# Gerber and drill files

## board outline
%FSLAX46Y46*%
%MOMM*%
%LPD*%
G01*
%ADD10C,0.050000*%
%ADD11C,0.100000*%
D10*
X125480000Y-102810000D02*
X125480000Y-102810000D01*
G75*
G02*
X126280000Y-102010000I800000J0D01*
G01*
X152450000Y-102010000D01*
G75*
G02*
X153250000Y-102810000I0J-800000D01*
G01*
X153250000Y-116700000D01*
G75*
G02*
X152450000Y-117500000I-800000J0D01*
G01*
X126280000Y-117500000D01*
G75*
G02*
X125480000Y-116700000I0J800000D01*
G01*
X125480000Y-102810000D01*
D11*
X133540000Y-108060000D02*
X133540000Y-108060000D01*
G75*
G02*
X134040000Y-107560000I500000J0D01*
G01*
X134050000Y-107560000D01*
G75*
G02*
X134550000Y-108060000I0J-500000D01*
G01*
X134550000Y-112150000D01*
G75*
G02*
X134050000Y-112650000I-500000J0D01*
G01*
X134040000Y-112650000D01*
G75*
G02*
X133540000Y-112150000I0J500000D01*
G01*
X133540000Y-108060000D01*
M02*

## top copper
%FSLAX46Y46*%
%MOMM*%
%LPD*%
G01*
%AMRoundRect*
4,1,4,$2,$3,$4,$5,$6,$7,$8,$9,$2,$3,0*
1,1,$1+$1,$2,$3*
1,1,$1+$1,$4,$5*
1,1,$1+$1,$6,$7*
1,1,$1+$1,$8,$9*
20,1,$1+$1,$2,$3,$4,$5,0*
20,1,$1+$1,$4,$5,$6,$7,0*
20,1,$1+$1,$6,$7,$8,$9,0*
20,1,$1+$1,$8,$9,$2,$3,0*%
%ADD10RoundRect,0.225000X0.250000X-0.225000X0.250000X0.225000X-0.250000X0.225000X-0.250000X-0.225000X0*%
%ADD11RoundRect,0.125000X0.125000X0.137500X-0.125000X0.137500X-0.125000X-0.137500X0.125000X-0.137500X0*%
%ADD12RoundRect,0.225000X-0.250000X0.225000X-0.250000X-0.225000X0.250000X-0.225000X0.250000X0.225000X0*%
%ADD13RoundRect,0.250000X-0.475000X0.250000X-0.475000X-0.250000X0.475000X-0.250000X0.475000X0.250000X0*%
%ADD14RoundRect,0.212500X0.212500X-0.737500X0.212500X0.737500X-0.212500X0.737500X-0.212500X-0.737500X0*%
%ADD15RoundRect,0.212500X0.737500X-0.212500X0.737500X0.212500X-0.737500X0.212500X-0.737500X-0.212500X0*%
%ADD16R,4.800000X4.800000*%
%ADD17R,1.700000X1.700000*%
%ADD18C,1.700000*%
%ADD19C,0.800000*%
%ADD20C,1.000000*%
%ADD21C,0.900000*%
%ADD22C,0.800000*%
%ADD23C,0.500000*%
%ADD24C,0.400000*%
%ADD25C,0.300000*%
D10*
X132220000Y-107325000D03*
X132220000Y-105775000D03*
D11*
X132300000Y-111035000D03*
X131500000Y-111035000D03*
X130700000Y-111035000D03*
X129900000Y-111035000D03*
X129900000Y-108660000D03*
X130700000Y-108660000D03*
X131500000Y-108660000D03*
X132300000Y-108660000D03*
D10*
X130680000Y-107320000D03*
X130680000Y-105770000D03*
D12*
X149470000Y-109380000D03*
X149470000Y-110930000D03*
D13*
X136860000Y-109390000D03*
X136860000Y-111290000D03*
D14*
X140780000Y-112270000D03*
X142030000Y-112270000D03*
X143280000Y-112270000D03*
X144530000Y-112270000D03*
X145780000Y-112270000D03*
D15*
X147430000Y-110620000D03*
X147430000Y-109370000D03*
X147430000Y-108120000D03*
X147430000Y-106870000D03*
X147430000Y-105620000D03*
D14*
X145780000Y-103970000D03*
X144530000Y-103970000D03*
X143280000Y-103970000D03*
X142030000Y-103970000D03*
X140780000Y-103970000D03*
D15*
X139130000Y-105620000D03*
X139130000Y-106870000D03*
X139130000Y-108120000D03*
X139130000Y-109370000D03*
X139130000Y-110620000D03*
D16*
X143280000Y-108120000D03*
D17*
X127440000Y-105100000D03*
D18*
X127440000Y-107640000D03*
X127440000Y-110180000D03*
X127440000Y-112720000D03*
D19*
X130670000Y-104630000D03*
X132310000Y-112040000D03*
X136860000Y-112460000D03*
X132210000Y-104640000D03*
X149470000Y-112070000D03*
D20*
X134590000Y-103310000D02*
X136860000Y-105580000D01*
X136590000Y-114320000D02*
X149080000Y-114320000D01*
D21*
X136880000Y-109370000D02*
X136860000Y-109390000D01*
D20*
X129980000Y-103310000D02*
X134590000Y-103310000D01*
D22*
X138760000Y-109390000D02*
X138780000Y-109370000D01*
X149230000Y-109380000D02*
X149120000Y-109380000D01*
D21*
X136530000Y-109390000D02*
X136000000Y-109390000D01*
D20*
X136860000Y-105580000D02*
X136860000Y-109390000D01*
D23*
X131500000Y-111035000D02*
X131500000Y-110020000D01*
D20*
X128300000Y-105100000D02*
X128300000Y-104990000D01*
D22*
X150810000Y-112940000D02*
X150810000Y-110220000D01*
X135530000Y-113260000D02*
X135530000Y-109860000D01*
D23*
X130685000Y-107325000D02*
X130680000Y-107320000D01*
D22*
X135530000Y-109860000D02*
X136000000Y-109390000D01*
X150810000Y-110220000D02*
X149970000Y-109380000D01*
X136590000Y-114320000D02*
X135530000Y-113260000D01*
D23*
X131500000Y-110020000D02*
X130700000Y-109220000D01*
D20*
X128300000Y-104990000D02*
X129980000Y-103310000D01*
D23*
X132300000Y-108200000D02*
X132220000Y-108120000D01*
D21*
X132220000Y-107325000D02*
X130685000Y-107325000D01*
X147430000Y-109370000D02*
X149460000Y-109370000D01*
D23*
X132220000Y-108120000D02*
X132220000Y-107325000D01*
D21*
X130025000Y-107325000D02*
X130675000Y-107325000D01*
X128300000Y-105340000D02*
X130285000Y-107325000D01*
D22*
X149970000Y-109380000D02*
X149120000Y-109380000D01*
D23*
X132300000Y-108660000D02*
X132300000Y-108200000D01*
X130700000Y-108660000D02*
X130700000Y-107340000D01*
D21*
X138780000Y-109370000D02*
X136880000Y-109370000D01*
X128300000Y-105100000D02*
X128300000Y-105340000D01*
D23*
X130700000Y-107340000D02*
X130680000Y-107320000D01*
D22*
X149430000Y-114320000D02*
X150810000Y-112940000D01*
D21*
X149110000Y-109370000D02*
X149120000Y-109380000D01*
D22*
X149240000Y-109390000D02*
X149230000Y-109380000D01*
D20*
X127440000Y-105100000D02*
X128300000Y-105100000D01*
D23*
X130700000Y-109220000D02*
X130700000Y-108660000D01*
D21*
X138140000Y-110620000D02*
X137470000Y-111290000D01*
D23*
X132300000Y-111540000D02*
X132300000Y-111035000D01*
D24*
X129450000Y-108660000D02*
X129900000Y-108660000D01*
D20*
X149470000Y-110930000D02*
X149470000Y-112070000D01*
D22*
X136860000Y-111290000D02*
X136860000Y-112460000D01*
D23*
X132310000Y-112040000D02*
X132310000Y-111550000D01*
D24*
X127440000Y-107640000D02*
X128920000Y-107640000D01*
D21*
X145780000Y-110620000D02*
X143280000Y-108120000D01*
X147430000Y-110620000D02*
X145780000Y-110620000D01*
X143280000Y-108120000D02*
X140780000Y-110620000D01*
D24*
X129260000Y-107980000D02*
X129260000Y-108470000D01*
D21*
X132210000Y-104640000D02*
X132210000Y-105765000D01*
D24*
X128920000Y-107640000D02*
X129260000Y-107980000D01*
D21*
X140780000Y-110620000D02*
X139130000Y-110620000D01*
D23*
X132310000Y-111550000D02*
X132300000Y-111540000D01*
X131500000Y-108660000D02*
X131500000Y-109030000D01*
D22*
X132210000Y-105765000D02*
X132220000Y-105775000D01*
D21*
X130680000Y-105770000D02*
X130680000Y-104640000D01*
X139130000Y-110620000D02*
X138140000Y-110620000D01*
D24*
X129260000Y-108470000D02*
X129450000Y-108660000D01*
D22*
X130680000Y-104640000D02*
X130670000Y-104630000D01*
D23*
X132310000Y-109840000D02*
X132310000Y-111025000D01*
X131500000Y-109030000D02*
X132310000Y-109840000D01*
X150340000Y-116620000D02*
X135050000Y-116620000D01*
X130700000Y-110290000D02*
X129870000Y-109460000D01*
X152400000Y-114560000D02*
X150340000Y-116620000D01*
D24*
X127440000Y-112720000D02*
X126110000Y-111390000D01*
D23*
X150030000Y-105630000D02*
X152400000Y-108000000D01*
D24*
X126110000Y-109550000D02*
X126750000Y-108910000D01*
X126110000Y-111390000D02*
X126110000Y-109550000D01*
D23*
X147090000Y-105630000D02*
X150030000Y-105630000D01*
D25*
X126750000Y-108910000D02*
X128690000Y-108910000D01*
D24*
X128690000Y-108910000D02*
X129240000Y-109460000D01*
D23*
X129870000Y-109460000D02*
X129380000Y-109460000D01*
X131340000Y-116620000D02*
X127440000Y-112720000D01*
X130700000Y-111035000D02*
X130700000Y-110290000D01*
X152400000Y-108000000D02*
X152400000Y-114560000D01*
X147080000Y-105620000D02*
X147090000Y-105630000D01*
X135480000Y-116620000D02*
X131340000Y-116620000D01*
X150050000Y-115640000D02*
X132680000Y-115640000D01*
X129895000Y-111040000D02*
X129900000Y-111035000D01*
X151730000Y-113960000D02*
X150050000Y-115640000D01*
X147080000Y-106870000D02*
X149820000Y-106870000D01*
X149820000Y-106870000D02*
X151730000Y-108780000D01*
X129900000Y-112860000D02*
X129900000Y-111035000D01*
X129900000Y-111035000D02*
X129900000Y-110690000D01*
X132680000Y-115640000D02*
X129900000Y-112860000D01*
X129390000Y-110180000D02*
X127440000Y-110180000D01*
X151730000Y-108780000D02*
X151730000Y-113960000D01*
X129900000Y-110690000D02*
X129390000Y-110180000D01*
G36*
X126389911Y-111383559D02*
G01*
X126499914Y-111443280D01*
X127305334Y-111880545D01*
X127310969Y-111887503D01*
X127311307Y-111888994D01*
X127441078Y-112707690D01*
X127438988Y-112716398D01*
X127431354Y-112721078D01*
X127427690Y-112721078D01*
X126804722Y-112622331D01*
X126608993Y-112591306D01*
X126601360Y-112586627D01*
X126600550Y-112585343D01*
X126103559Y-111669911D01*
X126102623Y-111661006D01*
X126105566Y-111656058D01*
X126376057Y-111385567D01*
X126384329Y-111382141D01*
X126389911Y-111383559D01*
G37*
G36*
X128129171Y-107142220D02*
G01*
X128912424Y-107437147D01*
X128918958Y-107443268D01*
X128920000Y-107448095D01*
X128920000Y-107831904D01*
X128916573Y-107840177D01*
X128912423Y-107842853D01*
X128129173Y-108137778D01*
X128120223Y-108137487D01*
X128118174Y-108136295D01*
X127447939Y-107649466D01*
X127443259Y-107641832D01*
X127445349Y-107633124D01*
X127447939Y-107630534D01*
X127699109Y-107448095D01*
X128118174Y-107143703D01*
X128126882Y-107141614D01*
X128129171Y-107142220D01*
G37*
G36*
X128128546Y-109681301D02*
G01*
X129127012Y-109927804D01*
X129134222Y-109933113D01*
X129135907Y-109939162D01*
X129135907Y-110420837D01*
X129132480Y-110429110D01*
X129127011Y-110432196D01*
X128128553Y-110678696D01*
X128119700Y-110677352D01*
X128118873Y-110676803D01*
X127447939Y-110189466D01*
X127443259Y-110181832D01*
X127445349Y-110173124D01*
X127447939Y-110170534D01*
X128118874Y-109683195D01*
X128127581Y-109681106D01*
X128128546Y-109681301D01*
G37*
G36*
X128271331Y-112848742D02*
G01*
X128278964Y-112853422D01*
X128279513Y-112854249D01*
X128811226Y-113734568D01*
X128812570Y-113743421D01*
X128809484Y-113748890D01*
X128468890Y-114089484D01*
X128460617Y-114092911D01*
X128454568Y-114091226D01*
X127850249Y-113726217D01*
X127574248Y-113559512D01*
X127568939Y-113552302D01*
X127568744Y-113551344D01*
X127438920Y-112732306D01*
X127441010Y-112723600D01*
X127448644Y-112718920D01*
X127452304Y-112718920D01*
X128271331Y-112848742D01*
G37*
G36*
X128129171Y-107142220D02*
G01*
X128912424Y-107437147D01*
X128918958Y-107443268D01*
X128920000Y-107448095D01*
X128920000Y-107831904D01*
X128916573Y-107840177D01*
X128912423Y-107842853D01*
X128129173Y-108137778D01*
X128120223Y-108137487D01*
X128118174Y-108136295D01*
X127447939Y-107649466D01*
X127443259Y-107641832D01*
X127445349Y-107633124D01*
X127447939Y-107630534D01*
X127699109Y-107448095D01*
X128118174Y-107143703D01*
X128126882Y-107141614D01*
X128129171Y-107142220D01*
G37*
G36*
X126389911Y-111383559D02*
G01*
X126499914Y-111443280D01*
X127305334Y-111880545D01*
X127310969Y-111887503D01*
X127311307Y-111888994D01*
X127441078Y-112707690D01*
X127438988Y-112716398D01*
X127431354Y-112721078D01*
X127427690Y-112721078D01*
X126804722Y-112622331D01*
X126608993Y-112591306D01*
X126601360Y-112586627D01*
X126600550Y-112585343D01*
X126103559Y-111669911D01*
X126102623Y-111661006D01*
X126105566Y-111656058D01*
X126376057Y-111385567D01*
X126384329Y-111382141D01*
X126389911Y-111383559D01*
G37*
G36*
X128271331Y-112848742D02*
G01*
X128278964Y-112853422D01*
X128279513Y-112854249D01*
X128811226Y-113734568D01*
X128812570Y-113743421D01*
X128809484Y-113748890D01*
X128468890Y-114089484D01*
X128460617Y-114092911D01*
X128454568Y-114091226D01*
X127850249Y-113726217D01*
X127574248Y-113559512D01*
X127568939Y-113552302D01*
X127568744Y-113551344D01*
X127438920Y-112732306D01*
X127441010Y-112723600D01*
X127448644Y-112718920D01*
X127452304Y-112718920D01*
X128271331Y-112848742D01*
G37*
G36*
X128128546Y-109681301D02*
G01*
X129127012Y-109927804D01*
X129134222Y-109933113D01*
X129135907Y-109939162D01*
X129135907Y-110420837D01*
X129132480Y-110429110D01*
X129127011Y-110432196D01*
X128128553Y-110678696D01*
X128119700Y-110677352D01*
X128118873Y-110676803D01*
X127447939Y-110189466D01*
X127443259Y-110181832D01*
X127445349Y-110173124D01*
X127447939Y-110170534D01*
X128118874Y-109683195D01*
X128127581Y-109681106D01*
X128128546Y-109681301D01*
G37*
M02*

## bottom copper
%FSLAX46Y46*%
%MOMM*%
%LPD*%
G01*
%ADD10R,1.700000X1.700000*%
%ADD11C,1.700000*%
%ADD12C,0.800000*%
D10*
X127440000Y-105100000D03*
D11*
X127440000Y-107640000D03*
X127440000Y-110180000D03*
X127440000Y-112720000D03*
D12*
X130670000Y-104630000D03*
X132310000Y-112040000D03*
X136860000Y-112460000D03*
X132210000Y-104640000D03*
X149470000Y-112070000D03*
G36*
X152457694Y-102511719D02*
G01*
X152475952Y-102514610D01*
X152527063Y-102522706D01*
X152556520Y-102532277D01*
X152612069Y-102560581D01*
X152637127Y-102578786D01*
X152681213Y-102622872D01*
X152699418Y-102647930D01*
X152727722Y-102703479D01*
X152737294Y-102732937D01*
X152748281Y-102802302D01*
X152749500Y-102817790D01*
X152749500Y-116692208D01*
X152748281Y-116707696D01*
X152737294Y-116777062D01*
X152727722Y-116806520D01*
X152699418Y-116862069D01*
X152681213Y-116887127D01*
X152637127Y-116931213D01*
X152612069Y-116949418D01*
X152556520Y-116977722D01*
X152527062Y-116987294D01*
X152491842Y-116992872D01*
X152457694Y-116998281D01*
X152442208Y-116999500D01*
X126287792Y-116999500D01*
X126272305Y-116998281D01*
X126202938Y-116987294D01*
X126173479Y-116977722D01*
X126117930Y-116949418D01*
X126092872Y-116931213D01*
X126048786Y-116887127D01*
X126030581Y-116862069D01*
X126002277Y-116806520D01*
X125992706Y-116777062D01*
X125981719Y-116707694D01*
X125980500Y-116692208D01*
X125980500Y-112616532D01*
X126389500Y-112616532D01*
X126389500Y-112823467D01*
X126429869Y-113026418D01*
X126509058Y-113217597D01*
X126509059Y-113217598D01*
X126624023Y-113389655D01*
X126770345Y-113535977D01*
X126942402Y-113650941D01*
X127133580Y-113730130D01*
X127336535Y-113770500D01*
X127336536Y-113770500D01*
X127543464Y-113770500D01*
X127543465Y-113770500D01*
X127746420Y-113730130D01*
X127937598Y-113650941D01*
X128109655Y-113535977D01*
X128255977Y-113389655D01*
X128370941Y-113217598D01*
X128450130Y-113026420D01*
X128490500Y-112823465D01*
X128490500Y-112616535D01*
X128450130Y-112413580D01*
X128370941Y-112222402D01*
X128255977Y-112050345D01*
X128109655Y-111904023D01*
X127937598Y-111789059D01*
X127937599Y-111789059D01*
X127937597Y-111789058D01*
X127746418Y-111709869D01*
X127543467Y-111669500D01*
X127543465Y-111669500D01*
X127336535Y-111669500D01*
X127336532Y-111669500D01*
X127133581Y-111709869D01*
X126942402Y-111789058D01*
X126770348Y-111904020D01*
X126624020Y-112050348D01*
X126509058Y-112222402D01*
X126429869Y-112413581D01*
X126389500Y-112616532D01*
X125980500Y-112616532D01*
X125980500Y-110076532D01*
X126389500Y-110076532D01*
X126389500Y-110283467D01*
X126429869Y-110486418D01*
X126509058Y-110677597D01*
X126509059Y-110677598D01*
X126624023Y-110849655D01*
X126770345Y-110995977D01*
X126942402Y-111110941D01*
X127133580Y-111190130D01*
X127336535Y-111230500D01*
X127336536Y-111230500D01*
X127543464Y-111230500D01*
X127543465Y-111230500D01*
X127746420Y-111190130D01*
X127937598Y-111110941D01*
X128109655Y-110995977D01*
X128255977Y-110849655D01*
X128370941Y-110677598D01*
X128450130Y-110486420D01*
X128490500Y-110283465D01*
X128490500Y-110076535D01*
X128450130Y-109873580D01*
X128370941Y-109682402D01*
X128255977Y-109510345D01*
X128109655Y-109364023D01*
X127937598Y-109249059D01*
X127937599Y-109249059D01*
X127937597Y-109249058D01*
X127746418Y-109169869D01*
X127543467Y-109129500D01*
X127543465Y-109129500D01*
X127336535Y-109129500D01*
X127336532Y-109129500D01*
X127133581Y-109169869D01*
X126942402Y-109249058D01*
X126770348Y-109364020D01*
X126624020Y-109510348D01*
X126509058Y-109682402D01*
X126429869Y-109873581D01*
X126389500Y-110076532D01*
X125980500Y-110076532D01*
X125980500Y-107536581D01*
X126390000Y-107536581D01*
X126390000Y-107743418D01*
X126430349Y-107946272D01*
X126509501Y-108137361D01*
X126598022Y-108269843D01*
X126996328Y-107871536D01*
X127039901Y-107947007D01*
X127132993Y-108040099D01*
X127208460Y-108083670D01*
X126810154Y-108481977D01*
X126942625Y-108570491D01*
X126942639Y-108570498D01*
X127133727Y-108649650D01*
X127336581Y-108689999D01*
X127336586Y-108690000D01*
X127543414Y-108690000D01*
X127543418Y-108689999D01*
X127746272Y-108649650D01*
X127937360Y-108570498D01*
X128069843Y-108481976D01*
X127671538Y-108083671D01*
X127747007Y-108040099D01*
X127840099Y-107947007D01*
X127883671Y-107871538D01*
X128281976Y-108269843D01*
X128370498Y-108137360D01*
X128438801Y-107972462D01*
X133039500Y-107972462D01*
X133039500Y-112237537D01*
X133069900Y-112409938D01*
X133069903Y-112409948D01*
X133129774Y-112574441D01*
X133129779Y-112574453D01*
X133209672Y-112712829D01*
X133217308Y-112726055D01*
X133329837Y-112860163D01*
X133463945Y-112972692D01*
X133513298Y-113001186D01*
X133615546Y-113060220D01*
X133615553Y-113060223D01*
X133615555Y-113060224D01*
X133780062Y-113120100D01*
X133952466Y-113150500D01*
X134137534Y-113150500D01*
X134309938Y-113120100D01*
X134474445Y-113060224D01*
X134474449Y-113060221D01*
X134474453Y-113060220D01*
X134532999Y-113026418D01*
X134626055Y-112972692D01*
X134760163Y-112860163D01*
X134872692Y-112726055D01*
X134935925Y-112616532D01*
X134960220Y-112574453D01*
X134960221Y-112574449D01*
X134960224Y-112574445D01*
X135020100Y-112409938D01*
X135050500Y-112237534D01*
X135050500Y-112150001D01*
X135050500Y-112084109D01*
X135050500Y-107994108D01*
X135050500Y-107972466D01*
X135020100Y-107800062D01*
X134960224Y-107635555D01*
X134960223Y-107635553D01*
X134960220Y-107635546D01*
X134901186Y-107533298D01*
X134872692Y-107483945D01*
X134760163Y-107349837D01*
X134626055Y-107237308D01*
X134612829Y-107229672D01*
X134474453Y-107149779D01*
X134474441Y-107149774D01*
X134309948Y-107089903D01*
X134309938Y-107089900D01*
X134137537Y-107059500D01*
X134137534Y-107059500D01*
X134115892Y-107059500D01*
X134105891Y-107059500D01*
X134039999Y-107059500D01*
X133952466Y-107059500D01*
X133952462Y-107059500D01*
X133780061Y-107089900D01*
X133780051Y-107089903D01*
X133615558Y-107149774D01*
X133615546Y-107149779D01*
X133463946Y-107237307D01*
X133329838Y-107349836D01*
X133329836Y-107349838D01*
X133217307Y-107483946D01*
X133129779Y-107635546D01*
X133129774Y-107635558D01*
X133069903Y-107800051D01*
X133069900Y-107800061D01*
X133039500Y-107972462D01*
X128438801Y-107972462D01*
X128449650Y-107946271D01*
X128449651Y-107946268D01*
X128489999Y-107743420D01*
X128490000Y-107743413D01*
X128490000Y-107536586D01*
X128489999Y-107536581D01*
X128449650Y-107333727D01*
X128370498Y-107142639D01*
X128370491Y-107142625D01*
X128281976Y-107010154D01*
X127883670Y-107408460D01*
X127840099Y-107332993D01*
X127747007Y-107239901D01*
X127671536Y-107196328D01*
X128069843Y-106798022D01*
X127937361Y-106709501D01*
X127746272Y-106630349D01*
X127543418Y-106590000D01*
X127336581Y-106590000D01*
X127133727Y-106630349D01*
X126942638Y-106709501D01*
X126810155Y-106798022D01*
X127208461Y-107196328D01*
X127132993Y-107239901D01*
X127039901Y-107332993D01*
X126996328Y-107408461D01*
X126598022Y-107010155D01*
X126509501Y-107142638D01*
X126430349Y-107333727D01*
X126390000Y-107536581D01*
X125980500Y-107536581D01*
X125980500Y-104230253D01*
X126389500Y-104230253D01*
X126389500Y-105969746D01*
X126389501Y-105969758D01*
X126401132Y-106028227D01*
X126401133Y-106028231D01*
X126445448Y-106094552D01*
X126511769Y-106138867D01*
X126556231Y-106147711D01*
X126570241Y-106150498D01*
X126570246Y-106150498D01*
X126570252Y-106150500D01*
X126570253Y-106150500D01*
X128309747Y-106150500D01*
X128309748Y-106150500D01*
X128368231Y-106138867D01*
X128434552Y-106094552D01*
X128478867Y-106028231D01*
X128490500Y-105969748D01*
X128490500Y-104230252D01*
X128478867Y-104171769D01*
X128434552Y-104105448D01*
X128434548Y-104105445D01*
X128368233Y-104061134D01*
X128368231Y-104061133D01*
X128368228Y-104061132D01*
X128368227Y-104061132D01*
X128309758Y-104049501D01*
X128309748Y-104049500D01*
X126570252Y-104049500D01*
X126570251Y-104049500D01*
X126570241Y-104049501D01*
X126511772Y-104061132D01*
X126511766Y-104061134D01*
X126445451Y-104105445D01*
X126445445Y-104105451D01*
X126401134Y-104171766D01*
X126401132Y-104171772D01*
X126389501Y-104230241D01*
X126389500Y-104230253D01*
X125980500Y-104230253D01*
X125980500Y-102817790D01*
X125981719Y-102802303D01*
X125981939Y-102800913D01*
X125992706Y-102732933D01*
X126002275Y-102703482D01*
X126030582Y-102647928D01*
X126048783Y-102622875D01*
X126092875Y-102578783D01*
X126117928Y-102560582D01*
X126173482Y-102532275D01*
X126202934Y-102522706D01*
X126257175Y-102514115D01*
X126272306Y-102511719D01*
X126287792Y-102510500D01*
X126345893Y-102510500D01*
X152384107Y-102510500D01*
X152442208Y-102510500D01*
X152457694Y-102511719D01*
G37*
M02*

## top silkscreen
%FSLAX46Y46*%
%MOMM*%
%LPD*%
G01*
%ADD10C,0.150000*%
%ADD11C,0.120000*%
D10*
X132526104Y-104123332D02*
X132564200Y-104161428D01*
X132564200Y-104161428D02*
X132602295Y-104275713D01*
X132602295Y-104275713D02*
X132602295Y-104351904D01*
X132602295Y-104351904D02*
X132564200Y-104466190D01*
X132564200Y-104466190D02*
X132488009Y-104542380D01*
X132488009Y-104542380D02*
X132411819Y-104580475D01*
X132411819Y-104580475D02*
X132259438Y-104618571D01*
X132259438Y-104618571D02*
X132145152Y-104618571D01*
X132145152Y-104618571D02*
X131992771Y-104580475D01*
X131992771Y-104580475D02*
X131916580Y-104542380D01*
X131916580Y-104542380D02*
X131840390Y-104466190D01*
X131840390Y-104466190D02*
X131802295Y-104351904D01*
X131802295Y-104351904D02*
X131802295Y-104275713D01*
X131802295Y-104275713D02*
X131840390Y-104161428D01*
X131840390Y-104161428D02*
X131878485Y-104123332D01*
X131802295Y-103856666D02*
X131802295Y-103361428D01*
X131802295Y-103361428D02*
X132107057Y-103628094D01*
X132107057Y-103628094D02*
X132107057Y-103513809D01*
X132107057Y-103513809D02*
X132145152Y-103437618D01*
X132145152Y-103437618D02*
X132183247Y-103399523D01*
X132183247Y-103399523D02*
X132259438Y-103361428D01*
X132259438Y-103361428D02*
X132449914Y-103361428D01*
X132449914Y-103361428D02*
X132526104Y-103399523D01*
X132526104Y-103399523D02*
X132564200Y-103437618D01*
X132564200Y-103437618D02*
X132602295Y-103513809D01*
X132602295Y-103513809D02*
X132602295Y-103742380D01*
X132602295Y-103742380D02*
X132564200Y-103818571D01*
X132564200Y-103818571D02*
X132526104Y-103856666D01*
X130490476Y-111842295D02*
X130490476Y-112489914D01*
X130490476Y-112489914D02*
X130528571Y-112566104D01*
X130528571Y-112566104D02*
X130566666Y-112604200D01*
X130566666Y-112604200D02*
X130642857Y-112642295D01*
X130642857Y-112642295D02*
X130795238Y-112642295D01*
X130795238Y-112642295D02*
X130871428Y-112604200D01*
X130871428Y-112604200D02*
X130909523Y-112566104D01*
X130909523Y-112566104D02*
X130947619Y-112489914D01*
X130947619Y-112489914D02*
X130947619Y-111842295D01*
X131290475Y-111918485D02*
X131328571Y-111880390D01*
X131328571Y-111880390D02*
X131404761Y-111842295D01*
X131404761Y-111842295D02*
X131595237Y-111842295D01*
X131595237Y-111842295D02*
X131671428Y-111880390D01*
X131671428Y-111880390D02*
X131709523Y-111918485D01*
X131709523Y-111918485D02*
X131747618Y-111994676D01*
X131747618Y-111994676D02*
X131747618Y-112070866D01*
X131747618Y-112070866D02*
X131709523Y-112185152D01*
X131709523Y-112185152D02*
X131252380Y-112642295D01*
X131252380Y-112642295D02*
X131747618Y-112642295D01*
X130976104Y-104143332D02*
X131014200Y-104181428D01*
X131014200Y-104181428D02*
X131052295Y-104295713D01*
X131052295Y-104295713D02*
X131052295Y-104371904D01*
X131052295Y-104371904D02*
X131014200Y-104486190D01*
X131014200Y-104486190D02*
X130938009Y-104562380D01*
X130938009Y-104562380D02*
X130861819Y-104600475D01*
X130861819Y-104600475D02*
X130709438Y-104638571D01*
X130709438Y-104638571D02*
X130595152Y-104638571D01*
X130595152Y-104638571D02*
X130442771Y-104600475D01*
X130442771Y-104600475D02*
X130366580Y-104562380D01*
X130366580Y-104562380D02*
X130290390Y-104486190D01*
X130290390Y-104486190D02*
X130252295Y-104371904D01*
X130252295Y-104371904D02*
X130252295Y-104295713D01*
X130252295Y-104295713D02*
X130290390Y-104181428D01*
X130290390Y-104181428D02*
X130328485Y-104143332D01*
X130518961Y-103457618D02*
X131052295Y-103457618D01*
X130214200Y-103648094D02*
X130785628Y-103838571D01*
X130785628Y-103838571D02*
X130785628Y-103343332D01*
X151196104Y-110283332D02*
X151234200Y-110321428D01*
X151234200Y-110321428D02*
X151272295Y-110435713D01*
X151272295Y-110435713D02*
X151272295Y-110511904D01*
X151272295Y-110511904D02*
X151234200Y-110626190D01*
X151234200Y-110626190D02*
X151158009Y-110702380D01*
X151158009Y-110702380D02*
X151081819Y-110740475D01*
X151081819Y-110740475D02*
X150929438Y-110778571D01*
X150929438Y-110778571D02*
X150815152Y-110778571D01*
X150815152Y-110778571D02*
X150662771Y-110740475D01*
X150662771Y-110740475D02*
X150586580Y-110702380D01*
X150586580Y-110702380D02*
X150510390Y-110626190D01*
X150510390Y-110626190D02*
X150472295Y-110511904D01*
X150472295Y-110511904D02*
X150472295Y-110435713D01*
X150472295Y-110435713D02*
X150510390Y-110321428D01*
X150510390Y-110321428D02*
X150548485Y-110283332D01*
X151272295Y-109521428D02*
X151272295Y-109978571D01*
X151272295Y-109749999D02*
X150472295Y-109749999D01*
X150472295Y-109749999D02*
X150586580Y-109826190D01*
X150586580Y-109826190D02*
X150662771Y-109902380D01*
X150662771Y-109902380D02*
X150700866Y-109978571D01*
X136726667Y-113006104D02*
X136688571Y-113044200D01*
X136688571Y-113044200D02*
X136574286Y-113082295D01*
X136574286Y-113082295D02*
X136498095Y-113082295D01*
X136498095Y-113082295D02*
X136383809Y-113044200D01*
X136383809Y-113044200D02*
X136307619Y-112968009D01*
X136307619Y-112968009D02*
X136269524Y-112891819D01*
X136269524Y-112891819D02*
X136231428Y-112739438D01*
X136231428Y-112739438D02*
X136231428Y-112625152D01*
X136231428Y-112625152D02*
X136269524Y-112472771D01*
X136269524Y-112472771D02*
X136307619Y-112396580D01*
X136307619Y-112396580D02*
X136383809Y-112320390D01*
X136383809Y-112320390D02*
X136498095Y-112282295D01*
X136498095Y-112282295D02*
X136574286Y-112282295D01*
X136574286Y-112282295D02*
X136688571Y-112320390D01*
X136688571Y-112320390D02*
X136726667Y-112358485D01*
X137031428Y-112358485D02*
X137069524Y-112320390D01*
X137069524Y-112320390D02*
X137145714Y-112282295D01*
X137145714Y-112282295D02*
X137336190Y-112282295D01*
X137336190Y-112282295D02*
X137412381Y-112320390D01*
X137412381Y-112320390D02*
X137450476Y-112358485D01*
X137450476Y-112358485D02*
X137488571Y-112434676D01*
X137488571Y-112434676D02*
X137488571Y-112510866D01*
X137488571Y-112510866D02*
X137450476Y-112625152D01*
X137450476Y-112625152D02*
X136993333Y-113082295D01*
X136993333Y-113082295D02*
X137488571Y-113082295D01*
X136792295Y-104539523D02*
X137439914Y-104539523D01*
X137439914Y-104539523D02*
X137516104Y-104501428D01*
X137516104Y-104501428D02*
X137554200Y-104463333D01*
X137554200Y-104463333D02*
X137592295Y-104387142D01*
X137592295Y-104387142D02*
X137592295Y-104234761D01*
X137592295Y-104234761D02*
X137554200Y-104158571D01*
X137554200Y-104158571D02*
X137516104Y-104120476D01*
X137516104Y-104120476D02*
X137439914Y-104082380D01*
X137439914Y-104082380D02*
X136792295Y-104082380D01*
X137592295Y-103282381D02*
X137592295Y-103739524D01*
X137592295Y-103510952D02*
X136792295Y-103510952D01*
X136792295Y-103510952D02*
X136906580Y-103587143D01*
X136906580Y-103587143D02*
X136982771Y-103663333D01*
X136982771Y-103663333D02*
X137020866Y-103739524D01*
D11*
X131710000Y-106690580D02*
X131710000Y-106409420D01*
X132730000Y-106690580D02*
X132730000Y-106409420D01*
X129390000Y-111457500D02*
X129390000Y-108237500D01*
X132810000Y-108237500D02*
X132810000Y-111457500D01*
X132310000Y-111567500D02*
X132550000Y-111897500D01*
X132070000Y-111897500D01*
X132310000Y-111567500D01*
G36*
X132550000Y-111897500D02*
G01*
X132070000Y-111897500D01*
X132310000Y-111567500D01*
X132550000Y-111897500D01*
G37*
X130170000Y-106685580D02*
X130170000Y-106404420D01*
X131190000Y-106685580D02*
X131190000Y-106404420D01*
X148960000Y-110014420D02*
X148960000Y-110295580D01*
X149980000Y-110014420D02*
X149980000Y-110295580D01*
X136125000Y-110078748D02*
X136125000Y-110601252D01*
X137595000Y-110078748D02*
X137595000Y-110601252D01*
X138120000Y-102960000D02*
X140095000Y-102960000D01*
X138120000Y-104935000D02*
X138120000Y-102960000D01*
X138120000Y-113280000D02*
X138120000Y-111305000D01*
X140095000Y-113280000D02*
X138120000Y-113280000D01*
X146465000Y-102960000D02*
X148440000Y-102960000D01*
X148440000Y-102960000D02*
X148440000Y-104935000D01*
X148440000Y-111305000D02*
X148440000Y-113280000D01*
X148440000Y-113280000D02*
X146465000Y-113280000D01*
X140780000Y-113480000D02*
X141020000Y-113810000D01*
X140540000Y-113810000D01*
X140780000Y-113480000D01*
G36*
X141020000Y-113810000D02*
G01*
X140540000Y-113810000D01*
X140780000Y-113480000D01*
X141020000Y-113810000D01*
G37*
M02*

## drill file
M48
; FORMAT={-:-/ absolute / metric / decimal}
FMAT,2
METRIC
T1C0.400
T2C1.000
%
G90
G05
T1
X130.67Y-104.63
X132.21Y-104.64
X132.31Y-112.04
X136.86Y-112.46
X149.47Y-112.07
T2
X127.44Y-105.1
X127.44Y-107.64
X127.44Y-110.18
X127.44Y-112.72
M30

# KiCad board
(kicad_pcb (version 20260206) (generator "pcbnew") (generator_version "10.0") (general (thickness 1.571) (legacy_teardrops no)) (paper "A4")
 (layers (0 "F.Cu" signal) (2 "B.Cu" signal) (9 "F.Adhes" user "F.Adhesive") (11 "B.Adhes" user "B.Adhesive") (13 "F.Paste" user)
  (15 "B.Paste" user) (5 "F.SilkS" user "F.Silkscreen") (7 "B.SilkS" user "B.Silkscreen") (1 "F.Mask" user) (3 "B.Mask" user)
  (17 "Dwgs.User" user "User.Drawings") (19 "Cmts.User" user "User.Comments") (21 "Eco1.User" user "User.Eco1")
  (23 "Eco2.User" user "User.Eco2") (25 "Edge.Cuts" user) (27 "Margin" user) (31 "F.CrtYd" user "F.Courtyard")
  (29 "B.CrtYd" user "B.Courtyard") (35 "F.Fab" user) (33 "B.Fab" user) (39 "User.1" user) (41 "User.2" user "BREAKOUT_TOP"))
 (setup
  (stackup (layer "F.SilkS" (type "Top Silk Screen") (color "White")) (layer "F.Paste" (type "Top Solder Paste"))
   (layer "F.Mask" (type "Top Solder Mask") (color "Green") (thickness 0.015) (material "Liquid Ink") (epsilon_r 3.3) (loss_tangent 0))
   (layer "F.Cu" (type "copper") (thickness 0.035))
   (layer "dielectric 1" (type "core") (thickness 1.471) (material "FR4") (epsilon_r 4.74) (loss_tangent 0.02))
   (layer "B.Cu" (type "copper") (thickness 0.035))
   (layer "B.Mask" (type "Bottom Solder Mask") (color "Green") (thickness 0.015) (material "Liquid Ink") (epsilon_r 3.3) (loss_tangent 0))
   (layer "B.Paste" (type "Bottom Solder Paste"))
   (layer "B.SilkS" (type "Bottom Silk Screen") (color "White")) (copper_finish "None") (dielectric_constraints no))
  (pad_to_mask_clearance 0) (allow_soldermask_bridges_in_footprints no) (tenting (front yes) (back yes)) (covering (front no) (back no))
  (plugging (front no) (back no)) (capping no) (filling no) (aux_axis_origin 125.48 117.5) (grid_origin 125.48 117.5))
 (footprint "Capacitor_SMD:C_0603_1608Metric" (layer "F.Cu") (at 132.22 106.55 90)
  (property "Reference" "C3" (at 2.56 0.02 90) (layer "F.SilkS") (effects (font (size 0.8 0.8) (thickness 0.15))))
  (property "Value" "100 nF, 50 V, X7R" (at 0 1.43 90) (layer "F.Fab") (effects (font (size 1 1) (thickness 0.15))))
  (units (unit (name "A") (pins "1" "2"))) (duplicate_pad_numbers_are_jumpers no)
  (fp_line (start -0.14058 -0.51) (end 0.14058 -0.51) (stroke (width 0.12) (type solid)) (layer "F.SilkS"))
  (fp_line (start -0.14058 0.51) (end 0.14058 0.51) (stroke (width 0.12) (type solid)) (layer "F.SilkS"))
  (pad "1" smd roundrect (at -0.775 0 90) (size 0.9 0.95) (layers "F.Cu" "F.Mask" "F.Paste") (roundrect_rratio 0.25) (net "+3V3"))
  (pad "2" smd roundrect (at 0.775 0 90) (size 0.9 0.95) (layers "F.Cu" "F.Mask" "F.Paste") (roundrect_rratio 0.25) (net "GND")))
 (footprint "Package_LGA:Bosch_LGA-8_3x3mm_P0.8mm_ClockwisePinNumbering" (layer "F.Cu") (at 131.1 109.8475 180)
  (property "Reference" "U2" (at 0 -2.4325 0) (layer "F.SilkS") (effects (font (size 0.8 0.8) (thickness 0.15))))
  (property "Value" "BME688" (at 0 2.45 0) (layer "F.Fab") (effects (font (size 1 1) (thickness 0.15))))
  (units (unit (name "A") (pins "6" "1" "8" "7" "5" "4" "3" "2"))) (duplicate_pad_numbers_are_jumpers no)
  (fp_line (start 1.71 -1.61) (end 1.71 1.61) (stroke (width 0.12) (type solid)) (layer "F.SilkS"))
  (fp_line (start -1.71 1.61) (end -1.71 -1.61) (stroke (width 0.12) (type solid)) (layer "F.SilkS"))
  (fp_poly (pts (xy -1.21 -1.72) (xy -1.45 -2.05) (xy -0.97 -2.05)) (stroke (width 0.12) (type solid)) (fill yes) (layer "F.SilkS"))
  (pad "1" smd roundrect (at -1.2 -1.1875 180) (size 0.5 0.525) (layers "F.Cu" "F.Mask" "F.Paste") (roundrect_rratio 0.25) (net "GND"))
  (pad "2" smd roundrect (at -0.4 -1.1875 180) (size 0.5 0.525) (layers "F.Cu" "F.Mask" "F.Paste") (roundrect_rratio 0.25) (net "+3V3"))
  (pad "3" smd roundrect (at 0.4 -1.1875 180) (size 0.5 0.525) (layers "F.Cu" "F.Mask" "F.Paste") (roundrect_rratio 0.25) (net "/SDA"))
  (pad "4" smd roundrect (at 1.2 -1.1875 180) (size 0.5 0.525) (layers "F.Cu" "F.Mask" "F.Paste") (roundrect_rratio 0.25) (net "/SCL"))
  (pad "5" smd roundrect (at 1.2 1.1875 180) (size 0.5 0.525) (layers "F.Cu" "F.Mask" "F.Paste") (roundrect_rratio 0.25) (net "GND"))
  (pad "6" smd roundrect (at 0.4 1.1875 180) (size 0.5 0.525) (layers "F.Cu" "F.Mask" "F.Paste") (roundrect_rratio 0.25) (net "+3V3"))
  (pad "7" smd roundrect (at -0.4 1.1875 180) (size 0.5 0.525) (layers "F.Cu" "F.Mask" "F.Paste") (roundrect_rratio 0.25) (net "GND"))
  (pad "8" smd roundrect (at -1.2 1.1875 180) (size 0.5 0.525) (layers "F.Cu" "F.Mask" "F.Paste") (roundrect_rratio 0.25) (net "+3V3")))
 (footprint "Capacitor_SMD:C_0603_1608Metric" (layer "F.Cu") (at 130.68 106.545 90)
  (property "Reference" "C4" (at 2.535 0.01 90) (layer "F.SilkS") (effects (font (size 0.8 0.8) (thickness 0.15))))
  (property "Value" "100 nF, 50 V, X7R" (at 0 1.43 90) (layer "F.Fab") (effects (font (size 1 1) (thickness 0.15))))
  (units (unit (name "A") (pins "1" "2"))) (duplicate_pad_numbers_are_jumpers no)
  (fp_line (start -0.14058 -0.51) (end 0.14058 -0.51) (stroke (width 0.12) (type solid)) (layer "F.SilkS"))
  (fp_line (start -0.14058 0.51) (end 0.14058 0.51) (stroke (width 0.12) (type solid)) (layer "F.SilkS"))
  (pad "1" smd roundrect (at -0.775 0 90) (size 0.9 0.95) (layers "F.Cu" "F.Mask" "F.Paste") (roundrect_rratio 0.25) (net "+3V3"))
  (pad "2" smd roundrect (at 0.775 0 90) (size 0.9 0.95) (layers "F.Cu" "F.Mask" "F.Paste") (roundrect_rratio 0.25) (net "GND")))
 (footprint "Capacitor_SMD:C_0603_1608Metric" (layer "F.Cu") (at 149.47 110.155 -90)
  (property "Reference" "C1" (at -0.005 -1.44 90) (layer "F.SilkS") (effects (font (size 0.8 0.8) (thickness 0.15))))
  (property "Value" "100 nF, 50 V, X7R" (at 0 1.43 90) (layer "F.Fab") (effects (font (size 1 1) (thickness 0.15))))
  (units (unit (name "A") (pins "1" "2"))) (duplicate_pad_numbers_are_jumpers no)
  (fp_line (start -0.14058 0.51) (end 0.14058 0.51) (stroke (width 0.12) (type solid)) (layer "F.SilkS"))
  (fp_line (start -0.14058 -0.51) (end 0.14058 -0.51) (stroke (width 0.12) (type solid)) (layer "F.SilkS"))
  (pad "1" smd roundrect (at -0.775 0 270) (size 0.9 0.95) (layers "F.Cu" "F.Mask" "F.Paste") (roundrect_rratio 0.25) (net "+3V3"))
  (pad "2" smd roundrect (at 0.775 0 270) (size 0.9 0.95) (layers "F.Cu" "F.Mask" "F.Paste") (roundrect_rratio 0.25) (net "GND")))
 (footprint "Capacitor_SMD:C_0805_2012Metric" (layer "F.Cu") (at 136.86 110.34 -90)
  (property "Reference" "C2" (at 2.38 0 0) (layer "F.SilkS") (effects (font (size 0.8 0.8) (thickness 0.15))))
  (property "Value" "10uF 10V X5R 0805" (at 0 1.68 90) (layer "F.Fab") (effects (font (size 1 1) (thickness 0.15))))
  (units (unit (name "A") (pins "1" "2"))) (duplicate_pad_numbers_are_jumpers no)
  (fp_line (start -0.261252 0.735) (end 0.261252 0.735) (stroke (width 0.12) (type solid)) (layer "F.SilkS"))
  (fp_line (start -0.261252 -0.735) (end 0.261252 -0.735) (stroke (width 0.12) (type solid)) (layer "F.SilkS"))
  (pad "1" smd roundrect (at -0.95 0 270) (size 1 1.45) (layers "F.Cu" "F.Mask" "F.Paste") (roundrect_rratio 0.25) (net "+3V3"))
  (pad "2" smd roundrect (at 0.95 0 270) (size 1 1.45) (layers "F.Cu" "F.Mask" "F.Paste") (roundrect_rratio 0.25) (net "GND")))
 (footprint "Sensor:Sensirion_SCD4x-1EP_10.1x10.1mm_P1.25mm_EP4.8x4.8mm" (layer "F.Cu") (at 143.28 108.12 90)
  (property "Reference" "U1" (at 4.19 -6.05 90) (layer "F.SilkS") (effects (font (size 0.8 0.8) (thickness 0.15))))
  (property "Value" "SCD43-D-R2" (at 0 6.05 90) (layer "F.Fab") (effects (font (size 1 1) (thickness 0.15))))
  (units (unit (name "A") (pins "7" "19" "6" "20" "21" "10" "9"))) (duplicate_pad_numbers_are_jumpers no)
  (fp_line (start 5.16 -5.16) (end 5.16 -3.185) (stroke (width 0.12) (type solid)) (layer "F.SilkS"))
  (fp_line (start 3.185 -5.16) (end 5.16 -5.16) (stroke (width 0.12) (type solid)) (layer "F.SilkS"))
  (fp_line (start -5.16 -5.16) (end -3.185 -5.16) (stroke (width 0.12) (type solid)) (layer "F.SilkS"))
  (fp_line (start -5.16 -3.185) (end -5.16 -5.16) (stroke (width 0.12) (type solid)) (layer "F.SilkS"))
  (fp_line (start 5.16 3.185) (end 5.16 5.16) (stroke (width 0.12) (type solid)) (layer "F.SilkS"))
  (fp_line (start 5.16 5.16) (end 3.185 5.16) (stroke (width 0.12) (type solid)) (layer "F.SilkS"))
  (fp_line (start -3.185 5.16) (end -5.16 5.16) (stroke (width 0.12) (type solid)) (layer "F.SilkS"))
  (fp_line (start -5.16 5.16) (end -5.16 3.185) (stroke (width 0.12) (type solid)) (layer "F.SilkS"))
  (fp_poly (pts (xy -5.36 -2.5) (xy -5.69 -2.26) (xy -5.69 -2.74)) (stroke (width 0.12) (type solid)) (fill yes) (layer "F.SilkS"))
  (pad "" smd roundrect (at -1.2 -1.2 90) (size 1.93 1.93) (layers "F.Paste") (roundrect_rratio 0.129534))
  (pad "" smd roundrect (at -1.2 1.2 90) (size 1.93 1.93) (layers "F.Paste") (roundrect_rratio 0.129534))
  (pad "" smd roundrect (at 1.2 -1.2 90) (size 1.93 1.93) (layers "F.Paste") (roundrect_rratio 0.129534))
  (pad "" smd roundrect (at 1.2 1.2 90) (size 1.93 1.93) (layers "F.Paste") (roundrect_rratio 0.129534))
  (pad "1" smd roundrect (at -4.15 -2.5 90) (size 1.9 0.85) (layers "F.Cu" "F.Mask" "F.Paste") (roundrect_rratio 0.25))
  (pad "2" smd roundrect (at -4.15 -1.25 90) (size 1.9 0.85) (layers "F.Cu" "F.Mask" "F.Paste") (roundrect_rratio 0.25))
  (pad "3" smd roundrect (at -4.15 0 90) (size 1.9 0.85) (layers "F.Cu" "F.Mask" "F.Paste") (roundrect_rratio 0.25))
  (pad "4" smd roundrect (at -4.15 1.25 90) (size 1.9 0.85) (layers "F.Cu" "F.Mask" "F.Paste") (roundrect_rratio 0.25))
  (pad "5" smd roundrect (at -4.15 2.5 90) (size 1.9 0.85) (layers "F.Cu" "F.Mask" "F.Paste") (roundrect_rratio 0.25))
  (pad "6" smd roundrect (at -2.5 4.15 90) (size 0.85 1.9) (layers "F.Cu" "F.Mask" "F.Paste") (roundrect_rratio 0.25) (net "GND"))
  (pad "7" smd roundrect (at -1.25 4.15 90) (size 0.85 1.9) (layers "F.Cu" "F.Mask" "F.Paste") (roundrect_rratio 0.25) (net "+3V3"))
  (pad "8" smd roundrect (at 0 4.15 90) (size 0.85 1.9) (layers "F.Cu" "F.Mask" "F.Paste") (roundrect_rratio 0.25))
  (pad "9" smd roundrect (at 1.25 4.15 90) (size 0.85 1.9) (layers "F.Cu" "F.Mask" "F.Paste") (roundrect_rratio 0.25) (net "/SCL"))
  (pad "10" smd roundrect (at 2.5 4.15 90) (size 0.85 1.9) (layers "F.Cu" "F.Mask" "F.Paste") (roundrect_rratio 0.25) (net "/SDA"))
  (pad "11" smd roundrect (at 4.15 2.5 90) (size 1.9 0.85) (layers "F.Cu" "F.Mask" "F.Paste") (roundrect_rratio 0.25))
  (pad "12" smd roundrect (at 4.15 1.25 90) (size 1.9 0.85) (layers "F.Cu" "F.Mask" "F.Paste") (roundrect_rratio 0.25))
  (pad "13" smd roundrect (at 4.15 0 90) (size 1.9 0.85) (layers "F.Cu" "F.Mask" "F.Paste") (roundrect_rratio 0.25))
  (pad "14" smd roundrect (at 4.15 -1.25 90) (size 1.9 0.85) (layers "F.Cu" "F.Mask" "F.Paste") (roundrect_rratio 0.25))
  (pad "15" smd roundrect (at 4.15 -2.5 90) (size 1.9 0.85) (layers "F.Cu" "F.Mask" "F.Paste") (roundrect_rratio 0.25))
  (pad "16" smd roundrect (at 2.5 -4.15 90) (size 0.85 1.9) (layers "F.Cu" "F.Mask" "F.Paste") (roundrect_rratio 0.25))
  (pad "17" smd roundrect (at 1.25 -4.15 90) (size 0.85 1.9) (layers "F.Cu" "F.Mask" "F.Paste") (roundrect_rratio 0.25))
  (pad "18" smd roundrect (at 0 -4.15 90) (size 0.85 1.9) (layers "F.Cu" "F.Mask" "F.Paste") (roundrect_rratio 0.25))
  (pad "19" smd roundrect (at -1.25 -4.15 90) (size 0.85 1.9) (layers "F.Cu" "F.Mask" "F.Paste") (roundrect_rratio 0.25) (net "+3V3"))
  (pad "20" smd roundrect (at -2.5 -4.15 90) (size 0.85 1.9) (layers "F.Cu" "F.Mask" "F.Paste") (roundrect_rratio 0.25) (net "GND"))
  (pad "21" smd rect (at 0 0 90) (size 4.8 4.8) (layers "F.Cu" "F.Mask") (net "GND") (zone_connect 2)))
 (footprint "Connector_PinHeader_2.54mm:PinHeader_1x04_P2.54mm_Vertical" (layer "B.Cu") (at 127.44 105.1 180)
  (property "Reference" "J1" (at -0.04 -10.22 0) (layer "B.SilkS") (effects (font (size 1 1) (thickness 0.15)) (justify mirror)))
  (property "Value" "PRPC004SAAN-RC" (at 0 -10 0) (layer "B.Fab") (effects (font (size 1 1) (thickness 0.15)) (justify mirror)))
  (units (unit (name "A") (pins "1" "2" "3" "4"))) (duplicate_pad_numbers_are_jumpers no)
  (pad "1" thru_hole rect (at 0 0 180) (size 1.7 1.7) (drill 1) (layers "*.Cu" "*.Mask") (remove_unused_layers no) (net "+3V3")
   (teardrops (best_length_ratio 0.5) (max_length 1) (best_width_ratio 1) (max_width 1) (curved_edges no) (filter_ratio 0.9) (enabled yes)
    (allow_two_segments no) (prefer_zone_connections yes)))
  (pad "2" thru_hole circle (at 0 -2.54 180) (size 1.7 1.7) (drill 1) (layers "*.Cu" "*.Mask") (remove_unused_layers no) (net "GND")
   (teardrops (best_length_ratio 0.5) (max_length 1) (best_width_ratio 1) (max_width 1) (curved_edges no) (filter_ratio 0.9) (enabled yes)
    (allow_two_segments no) (prefer_zone_connections yes)))
  (pad "3" thru_hole circle (at 0 -5.08 180) (size 1.7 1.7) (drill 1) (layers "*.Cu" "*.Mask") (remove_unused_layers no) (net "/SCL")
   (teardrops (best_length_ratio 0.5) (max_length 1) (best_width_ratio 1) (max_width 1) (curved_edges no) (filter_ratio 0.9) (enabled yes)
    (allow_two_segments no) (prefer_zone_connections yes)))
  (pad "4" thru_hole circle (at 0 -7.62 180) (size 1.7 1.7) (drill 1) (layers "*.Cu" "*.Mask") (remove_unused_layers no) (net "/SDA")
   (teardrops (best_length_ratio 0.5) (max_length 1) (best_width_ratio 1) (max_width 1) (curved_edges no) (filter_ratio 0.9) (enabled yes)
    (allow_two_segments no) (prefer_zone_connections yes))))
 (gr_rect (start 125.48 102.01) (end 153.25 117.5) (radius 0.8) (stroke (width 0.05) (type solid)) (fill no) (layer "Edge.Cuts"))
 (gr_rect (start 133.54 107.56) (end 134.55 112.65) (radius 0.5) (stroke (width 0.1) (type solid)) (fill no) (layer "Edge.Cuts"))
 (segment (start 134.59 103.31) (end 136.86 105.58) (width 1) (layer "F.Cu") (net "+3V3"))
 (segment (start 136.59 114.32) (end 149.08 114.32) (width 1) (layer "F.Cu") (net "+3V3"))
 (segment (start 136.88 109.37) (end 136.86 109.39) (width 0.9) (layer "F.Cu") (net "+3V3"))
 (segment (start 129.98 103.31) (end 134.59 103.31) (width 1) (layer "F.Cu") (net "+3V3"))
 (segment (start 138.76 109.39) (end 138.78 109.37) (width 0.8) (layer "F.Cu") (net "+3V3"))
 (segment (start 149.23 109.38) (end 149.12 109.38) (width 0.8) (layer "F.Cu") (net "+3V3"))
 (segment (start 136.53 109.39) (end 136 109.39) (width 0.9) (layer "F.Cu") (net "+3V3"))
 (segment (start 136.86 105.58) (end 136.86 109.39) (width 1) (layer "F.Cu") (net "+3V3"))
 (segment (start 131.5 111.035) (end 131.5 110.02) (width 0.5) (layer "F.Cu") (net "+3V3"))
 (segment (start 128.3 105.1) (end 128.3 104.99) (width 1) (layer "F.Cu") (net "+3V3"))
 (segment (start 150.81 112.94) (end 150.81 110.22) (width 0.8) (layer "F.Cu") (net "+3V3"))
 (segment (start 135.53 113.26) (end 135.53 109.86) (width 0.8) (layer "F.Cu") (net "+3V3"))
 (segment (start 130.685 107.325) (end 130.68 107.32) (width 0.5) (layer "F.Cu") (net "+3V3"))
 (segment (start 135.53 109.86) (end 136 109.39) (width 0.8) (layer "F.Cu") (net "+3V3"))
 (segment (start 150.81 110.22) (end 149.97 109.38) (width 0.8) (layer "F.Cu") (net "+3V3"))
 (segment (start 136.59 114.32) (end 135.53 113.26) (width 0.8) (layer "F.Cu") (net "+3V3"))
 (segment (start 131.5 110.02) (end 130.7 109.22) (width 0.5) (layer "F.Cu") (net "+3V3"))
 (segment (start 128.3 104.99) (end 129.98 103.31) (width 1) (layer "F.Cu") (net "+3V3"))
 (segment (start 132.3 108.2) (end 132.22 108.12) (width 0.5) (layer "F.Cu") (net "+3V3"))
 (segment (start 132.22 107.325) (end 130.685 107.325) (width 0.9) (layer "F.Cu") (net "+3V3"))
 (segment (start 147.43 109.37) (end 149.46 109.37) (width 0.9) (layer "F.Cu") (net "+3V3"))
 (segment (start 132.22 108.12) (end 132.22 107.325) (width 0.5) (layer "F.Cu") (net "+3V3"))
 (segment (start 130.025 107.325) (end 130.675 107.325) (width 0.9) (layer "F.Cu") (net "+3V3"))
 (segment (start 128.3 105.34) (end 130.285 107.325) (width 0.9) (layer "F.Cu") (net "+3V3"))
 (segment (start 149.97 109.38) (end 149.12 109.38) (width 0.8) (layer "F.Cu") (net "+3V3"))
 (segment (start 132.3 108.66) (end 132.3 108.2) (width 0.5) (layer "F.Cu") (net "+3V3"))
 (segment (start 130.7 108.66) (end 130.7 107.34) (width 0.5) (layer "F.Cu") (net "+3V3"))
 (segment (start 138.78 109.37) (end 136.88 109.37) (width 0.9) (layer "F.Cu") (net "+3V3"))
 (segment (start 128.3 105.1) (end 128.3 105.34) (width 0.9) (layer "F.Cu") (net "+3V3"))
 (segment (start 130.7 107.34) (end 130.68 107.32) (width 0.5) (layer "F.Cu") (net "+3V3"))
 (segment (start 149.43 114.32) (end 150.81 112.94) (width 0.8) (layer "F.Cu") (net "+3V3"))
 (segment (start 149.11 109.37) (end 149.12 109.38) (width 0.9) (layer "F.Cu") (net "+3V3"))
 (segment (start 149.24 109.39) (end 149.23 109.38) (width 0.8) (layer "F.Cu") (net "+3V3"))
 (segment (start 127.44 105.1) (end 128.3 105.1) (width 1) (layer "F.Cu") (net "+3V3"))
 (segment (start 130.7 109.22) (end 130.7 108.66) (width 0.5) (layer "F.Cu") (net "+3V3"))
 (segment (start 138.14 110.62) (end 137.47 111.29) (width 0.9) (layer "F.Cu") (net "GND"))
 (segment (start 132.3 111.54) (end 132.3 111.035) (width 0.5) (layer "F.Cu") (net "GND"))
 (segment (start 129.45 108.66) (end 129.9 108.66) (width 0.4) (layer "F.Cu") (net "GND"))
 (segment (start 149.47 110.93) (end 149.47 112.07) (width 1) (layer "F.Cu") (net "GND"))
 (segment (start 136.86 111.29) (end 136.86 112.46) (width 0.8) (layer "F.Cu") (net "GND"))
 (segment (start 132.31 112.04) (end 132.31 111.55) (width 0.5) (layer "F.Cu") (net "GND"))
 (segment (start 127.44 107.64) (end 128.92 107.64) (width 0.4) (layer "F.Cu") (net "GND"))
 (segment (start 145.78 110.62) (end 143.28 108.12) (width 0.9) (layer "F.Cu") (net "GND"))
 (segment (start 147.43 110.62) (end 145.78 110.62) (width 0.9) (layer "F.Cu") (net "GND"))
 (segment (start 143.28 108.12) (end 140.78 110.62) (width 0.9) (layer "F.Cu") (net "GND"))
 (segment (start 129.26 107.98) (end 129.26 108.47) (width 0.4) (layer "F.Cu") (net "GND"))
 (segment (start 132.21 104.64) (end 132.21 105.765) (width 0.9) (layer "F.Cu") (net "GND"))
 (segment (start 128.92 107.64) (end 129.26 107.98) (width 0.4) (layer "F.Cu") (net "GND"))
 (segment (start 140.78 110.62) (end 139.13 110.62) (width 0.9) (layer "F.Cu") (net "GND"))
 (segment (start 132.31 111.55) (end 132.3 111.54) (width 0.5) (layer "F.Cu") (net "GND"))
 (segment (start 131.5 108.66) (end 131.5 109.03) (width 0.5) (layer "F.Cu") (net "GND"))
 (segment (start 132.21 105.765) (end 132.22 105.775) (width 0.8) (layer "F.Cu") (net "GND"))
 (segment (start 130.68 105.77) (end 130.68 104.64) (width 0.9) (layer "F.Cu") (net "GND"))
 (segment (start 139.13 110.62) (end 138.14 110.62) (width 0.9) (layer "F.Cu") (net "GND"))
 (segment (start 129.26 108.47) (end 129.45 108.66) (width 0.4) (layer "F.Cu") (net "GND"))
 (segment (start 130.68 104.64) (end 130.67 104.63) (width 0.8) (layer "F.Cu") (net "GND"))
 (segment (start 132.31 109.84) (end 132.31 111.025) (width 0.5) (layer "F.Cu") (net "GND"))
 (segment (start 131.5 109.03) (end 132.31 109.84) (width 0.5) (layer "F.Cu") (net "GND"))
 (via (at 130.67 104.63) (size 0.8) (drill 0.4) (layers "F.Cu" "B.Cu") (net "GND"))
 (via (at 132.31 112.04) (size 0.8) (drill 0.4) (layers "F.Cu" "B.Cu") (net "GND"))
 (via (at 136.86 112.46) (size 0.8) (drill 0.4) (layers "F.Cu" "B.Cu") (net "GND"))
 (via (at 132.21 104.64) (size 0.8) (drill 0.4) (layers "F.Cu" "B.Cu") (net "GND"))
 (via (at 149.47 112.07) (size 0.8) (drill 0.4) (layers "F.Cu" "B.Cu") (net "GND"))
 (segment (start 150.34 116.62) (end 135.05 116.62) (width 0.5) (layer "F.Cu") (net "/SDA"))
 (segment (start 130.7 110.29) (end 129.87 109.46) (width 0.5) (layer "F.Cu") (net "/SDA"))
 (segment (start 152.4 114.56) (end 150.34 116.62) (width 0.5) (layer "F.Cu") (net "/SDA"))
 (segment (start 127.44 112.72) (end 126.11 111.39) (width 0.4) (layer "F.Cu") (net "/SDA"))
 (segment (start 150.03 105.63) (end 152.4 108) (width 0.5) (layer "F.Cu") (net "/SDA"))
 (segment (start 126.11 109.55) (end 126.75 108.91) (width 0.4) (layer "F.Cu") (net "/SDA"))
 (segment (start 126.11 111.39) (end 126.11 109.55) (width 0.4) (layer "F.Cu") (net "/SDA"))
 (segment (start 147.09 105.63) (end 150.03 105.63) (width 0.5) (layer "F.Cu") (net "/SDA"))
 (segment (start 126.75 108.91) (end 128.69 108.91) (width 0.3) (layer "F.Cu") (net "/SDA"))
 (segment (start 128.69 108.91) (end 129.24 109.46) (width 0.4) (layer "F.Cu") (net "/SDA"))
 (segment (start 129.87 109.46) (end 129.38 109.46) (width 0.5) (layer "F.Cu") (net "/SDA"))
 (segment (start 131.34 116.62) (end 127.44 112.72) (width 0.5) (layer "F.Cu") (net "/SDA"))
 (segment (start 130.7 111.035) (end 130.7 110.29) (width 0.5) (layer "F.Cu") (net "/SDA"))
 (segment (start 152.4 108) (end 152.4 114.56) (width 0.5) (layer "F.Cu") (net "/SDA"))
 (segment (start 147.08 105.62) (end 147.09 105.63) (width 0.5) (layer "F.Cu") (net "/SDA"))
 (segment (start 135.48 116.62) (end 131.34 116.62) (width 0.5) (layer "F.Cu") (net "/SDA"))
 (segment (start 150.05 115.64) (end 132.68 115.64) (width 0.5) (layer "F.Cu") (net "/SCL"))
 (segment (start 129.895 111.04) (end 129.9 111.035) (width 0.5) (layer "F.Cu") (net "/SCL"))
 (segment (start 151.73 113.96) (end 150.05 115.64) (width 0.5) (layer "F.Cu") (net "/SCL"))
 (segment (start 147.08 106.87) (end 149.82 106.87) (width 0.5) (layer "F.Cu") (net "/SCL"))
 (segment (start 149.82 106.87) (end 151.73 108.78) (width 0.5) (layer "F.Cu") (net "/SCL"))
 (segment (start 129.9 112.86) (end 129.9 111.035) (width 0.5) (layer "F.Cu") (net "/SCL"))
 (segment (start 129.9 111.035) (end 129.9 110.69) (width 0.5) (layer "F.Cu") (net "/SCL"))
 (segment (start 132.68 115.64) (end 129.9 112.86) (width 0.5) (layer "F.Cu") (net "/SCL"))
 (segment (start 129.39 110.18) (end 127.44 110.18) (width 0.5) (layer "F.Cu") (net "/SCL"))
 (segment (start 151.73 108.78) (end 151.73 113.96) (width 0.5) (layer "F.Cu") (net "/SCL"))
 (segment (start 129.9 110.69) (end 129.39 110.18) (width 0.5) (layer "F.Cu") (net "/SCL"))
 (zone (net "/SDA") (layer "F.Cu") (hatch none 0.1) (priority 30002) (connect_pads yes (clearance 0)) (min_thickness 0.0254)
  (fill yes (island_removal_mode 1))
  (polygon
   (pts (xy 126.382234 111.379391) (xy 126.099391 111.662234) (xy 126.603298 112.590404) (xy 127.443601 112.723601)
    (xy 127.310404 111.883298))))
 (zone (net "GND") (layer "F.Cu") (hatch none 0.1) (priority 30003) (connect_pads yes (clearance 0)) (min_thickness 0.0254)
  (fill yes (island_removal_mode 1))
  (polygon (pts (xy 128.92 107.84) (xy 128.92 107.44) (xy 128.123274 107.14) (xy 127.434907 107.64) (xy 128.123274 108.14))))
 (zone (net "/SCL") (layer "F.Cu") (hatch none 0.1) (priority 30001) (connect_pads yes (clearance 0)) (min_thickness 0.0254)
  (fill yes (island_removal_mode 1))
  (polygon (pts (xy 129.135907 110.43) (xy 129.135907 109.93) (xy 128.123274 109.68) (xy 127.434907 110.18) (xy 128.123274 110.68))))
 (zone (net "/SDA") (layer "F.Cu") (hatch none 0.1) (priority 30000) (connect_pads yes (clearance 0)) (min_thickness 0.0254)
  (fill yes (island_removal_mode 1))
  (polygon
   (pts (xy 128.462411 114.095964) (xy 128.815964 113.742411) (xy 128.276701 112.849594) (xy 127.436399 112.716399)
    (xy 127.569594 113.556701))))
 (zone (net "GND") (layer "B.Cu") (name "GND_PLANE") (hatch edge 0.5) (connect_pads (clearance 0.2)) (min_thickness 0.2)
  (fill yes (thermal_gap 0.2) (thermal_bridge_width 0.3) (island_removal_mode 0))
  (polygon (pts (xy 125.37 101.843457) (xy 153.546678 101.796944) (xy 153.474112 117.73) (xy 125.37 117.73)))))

